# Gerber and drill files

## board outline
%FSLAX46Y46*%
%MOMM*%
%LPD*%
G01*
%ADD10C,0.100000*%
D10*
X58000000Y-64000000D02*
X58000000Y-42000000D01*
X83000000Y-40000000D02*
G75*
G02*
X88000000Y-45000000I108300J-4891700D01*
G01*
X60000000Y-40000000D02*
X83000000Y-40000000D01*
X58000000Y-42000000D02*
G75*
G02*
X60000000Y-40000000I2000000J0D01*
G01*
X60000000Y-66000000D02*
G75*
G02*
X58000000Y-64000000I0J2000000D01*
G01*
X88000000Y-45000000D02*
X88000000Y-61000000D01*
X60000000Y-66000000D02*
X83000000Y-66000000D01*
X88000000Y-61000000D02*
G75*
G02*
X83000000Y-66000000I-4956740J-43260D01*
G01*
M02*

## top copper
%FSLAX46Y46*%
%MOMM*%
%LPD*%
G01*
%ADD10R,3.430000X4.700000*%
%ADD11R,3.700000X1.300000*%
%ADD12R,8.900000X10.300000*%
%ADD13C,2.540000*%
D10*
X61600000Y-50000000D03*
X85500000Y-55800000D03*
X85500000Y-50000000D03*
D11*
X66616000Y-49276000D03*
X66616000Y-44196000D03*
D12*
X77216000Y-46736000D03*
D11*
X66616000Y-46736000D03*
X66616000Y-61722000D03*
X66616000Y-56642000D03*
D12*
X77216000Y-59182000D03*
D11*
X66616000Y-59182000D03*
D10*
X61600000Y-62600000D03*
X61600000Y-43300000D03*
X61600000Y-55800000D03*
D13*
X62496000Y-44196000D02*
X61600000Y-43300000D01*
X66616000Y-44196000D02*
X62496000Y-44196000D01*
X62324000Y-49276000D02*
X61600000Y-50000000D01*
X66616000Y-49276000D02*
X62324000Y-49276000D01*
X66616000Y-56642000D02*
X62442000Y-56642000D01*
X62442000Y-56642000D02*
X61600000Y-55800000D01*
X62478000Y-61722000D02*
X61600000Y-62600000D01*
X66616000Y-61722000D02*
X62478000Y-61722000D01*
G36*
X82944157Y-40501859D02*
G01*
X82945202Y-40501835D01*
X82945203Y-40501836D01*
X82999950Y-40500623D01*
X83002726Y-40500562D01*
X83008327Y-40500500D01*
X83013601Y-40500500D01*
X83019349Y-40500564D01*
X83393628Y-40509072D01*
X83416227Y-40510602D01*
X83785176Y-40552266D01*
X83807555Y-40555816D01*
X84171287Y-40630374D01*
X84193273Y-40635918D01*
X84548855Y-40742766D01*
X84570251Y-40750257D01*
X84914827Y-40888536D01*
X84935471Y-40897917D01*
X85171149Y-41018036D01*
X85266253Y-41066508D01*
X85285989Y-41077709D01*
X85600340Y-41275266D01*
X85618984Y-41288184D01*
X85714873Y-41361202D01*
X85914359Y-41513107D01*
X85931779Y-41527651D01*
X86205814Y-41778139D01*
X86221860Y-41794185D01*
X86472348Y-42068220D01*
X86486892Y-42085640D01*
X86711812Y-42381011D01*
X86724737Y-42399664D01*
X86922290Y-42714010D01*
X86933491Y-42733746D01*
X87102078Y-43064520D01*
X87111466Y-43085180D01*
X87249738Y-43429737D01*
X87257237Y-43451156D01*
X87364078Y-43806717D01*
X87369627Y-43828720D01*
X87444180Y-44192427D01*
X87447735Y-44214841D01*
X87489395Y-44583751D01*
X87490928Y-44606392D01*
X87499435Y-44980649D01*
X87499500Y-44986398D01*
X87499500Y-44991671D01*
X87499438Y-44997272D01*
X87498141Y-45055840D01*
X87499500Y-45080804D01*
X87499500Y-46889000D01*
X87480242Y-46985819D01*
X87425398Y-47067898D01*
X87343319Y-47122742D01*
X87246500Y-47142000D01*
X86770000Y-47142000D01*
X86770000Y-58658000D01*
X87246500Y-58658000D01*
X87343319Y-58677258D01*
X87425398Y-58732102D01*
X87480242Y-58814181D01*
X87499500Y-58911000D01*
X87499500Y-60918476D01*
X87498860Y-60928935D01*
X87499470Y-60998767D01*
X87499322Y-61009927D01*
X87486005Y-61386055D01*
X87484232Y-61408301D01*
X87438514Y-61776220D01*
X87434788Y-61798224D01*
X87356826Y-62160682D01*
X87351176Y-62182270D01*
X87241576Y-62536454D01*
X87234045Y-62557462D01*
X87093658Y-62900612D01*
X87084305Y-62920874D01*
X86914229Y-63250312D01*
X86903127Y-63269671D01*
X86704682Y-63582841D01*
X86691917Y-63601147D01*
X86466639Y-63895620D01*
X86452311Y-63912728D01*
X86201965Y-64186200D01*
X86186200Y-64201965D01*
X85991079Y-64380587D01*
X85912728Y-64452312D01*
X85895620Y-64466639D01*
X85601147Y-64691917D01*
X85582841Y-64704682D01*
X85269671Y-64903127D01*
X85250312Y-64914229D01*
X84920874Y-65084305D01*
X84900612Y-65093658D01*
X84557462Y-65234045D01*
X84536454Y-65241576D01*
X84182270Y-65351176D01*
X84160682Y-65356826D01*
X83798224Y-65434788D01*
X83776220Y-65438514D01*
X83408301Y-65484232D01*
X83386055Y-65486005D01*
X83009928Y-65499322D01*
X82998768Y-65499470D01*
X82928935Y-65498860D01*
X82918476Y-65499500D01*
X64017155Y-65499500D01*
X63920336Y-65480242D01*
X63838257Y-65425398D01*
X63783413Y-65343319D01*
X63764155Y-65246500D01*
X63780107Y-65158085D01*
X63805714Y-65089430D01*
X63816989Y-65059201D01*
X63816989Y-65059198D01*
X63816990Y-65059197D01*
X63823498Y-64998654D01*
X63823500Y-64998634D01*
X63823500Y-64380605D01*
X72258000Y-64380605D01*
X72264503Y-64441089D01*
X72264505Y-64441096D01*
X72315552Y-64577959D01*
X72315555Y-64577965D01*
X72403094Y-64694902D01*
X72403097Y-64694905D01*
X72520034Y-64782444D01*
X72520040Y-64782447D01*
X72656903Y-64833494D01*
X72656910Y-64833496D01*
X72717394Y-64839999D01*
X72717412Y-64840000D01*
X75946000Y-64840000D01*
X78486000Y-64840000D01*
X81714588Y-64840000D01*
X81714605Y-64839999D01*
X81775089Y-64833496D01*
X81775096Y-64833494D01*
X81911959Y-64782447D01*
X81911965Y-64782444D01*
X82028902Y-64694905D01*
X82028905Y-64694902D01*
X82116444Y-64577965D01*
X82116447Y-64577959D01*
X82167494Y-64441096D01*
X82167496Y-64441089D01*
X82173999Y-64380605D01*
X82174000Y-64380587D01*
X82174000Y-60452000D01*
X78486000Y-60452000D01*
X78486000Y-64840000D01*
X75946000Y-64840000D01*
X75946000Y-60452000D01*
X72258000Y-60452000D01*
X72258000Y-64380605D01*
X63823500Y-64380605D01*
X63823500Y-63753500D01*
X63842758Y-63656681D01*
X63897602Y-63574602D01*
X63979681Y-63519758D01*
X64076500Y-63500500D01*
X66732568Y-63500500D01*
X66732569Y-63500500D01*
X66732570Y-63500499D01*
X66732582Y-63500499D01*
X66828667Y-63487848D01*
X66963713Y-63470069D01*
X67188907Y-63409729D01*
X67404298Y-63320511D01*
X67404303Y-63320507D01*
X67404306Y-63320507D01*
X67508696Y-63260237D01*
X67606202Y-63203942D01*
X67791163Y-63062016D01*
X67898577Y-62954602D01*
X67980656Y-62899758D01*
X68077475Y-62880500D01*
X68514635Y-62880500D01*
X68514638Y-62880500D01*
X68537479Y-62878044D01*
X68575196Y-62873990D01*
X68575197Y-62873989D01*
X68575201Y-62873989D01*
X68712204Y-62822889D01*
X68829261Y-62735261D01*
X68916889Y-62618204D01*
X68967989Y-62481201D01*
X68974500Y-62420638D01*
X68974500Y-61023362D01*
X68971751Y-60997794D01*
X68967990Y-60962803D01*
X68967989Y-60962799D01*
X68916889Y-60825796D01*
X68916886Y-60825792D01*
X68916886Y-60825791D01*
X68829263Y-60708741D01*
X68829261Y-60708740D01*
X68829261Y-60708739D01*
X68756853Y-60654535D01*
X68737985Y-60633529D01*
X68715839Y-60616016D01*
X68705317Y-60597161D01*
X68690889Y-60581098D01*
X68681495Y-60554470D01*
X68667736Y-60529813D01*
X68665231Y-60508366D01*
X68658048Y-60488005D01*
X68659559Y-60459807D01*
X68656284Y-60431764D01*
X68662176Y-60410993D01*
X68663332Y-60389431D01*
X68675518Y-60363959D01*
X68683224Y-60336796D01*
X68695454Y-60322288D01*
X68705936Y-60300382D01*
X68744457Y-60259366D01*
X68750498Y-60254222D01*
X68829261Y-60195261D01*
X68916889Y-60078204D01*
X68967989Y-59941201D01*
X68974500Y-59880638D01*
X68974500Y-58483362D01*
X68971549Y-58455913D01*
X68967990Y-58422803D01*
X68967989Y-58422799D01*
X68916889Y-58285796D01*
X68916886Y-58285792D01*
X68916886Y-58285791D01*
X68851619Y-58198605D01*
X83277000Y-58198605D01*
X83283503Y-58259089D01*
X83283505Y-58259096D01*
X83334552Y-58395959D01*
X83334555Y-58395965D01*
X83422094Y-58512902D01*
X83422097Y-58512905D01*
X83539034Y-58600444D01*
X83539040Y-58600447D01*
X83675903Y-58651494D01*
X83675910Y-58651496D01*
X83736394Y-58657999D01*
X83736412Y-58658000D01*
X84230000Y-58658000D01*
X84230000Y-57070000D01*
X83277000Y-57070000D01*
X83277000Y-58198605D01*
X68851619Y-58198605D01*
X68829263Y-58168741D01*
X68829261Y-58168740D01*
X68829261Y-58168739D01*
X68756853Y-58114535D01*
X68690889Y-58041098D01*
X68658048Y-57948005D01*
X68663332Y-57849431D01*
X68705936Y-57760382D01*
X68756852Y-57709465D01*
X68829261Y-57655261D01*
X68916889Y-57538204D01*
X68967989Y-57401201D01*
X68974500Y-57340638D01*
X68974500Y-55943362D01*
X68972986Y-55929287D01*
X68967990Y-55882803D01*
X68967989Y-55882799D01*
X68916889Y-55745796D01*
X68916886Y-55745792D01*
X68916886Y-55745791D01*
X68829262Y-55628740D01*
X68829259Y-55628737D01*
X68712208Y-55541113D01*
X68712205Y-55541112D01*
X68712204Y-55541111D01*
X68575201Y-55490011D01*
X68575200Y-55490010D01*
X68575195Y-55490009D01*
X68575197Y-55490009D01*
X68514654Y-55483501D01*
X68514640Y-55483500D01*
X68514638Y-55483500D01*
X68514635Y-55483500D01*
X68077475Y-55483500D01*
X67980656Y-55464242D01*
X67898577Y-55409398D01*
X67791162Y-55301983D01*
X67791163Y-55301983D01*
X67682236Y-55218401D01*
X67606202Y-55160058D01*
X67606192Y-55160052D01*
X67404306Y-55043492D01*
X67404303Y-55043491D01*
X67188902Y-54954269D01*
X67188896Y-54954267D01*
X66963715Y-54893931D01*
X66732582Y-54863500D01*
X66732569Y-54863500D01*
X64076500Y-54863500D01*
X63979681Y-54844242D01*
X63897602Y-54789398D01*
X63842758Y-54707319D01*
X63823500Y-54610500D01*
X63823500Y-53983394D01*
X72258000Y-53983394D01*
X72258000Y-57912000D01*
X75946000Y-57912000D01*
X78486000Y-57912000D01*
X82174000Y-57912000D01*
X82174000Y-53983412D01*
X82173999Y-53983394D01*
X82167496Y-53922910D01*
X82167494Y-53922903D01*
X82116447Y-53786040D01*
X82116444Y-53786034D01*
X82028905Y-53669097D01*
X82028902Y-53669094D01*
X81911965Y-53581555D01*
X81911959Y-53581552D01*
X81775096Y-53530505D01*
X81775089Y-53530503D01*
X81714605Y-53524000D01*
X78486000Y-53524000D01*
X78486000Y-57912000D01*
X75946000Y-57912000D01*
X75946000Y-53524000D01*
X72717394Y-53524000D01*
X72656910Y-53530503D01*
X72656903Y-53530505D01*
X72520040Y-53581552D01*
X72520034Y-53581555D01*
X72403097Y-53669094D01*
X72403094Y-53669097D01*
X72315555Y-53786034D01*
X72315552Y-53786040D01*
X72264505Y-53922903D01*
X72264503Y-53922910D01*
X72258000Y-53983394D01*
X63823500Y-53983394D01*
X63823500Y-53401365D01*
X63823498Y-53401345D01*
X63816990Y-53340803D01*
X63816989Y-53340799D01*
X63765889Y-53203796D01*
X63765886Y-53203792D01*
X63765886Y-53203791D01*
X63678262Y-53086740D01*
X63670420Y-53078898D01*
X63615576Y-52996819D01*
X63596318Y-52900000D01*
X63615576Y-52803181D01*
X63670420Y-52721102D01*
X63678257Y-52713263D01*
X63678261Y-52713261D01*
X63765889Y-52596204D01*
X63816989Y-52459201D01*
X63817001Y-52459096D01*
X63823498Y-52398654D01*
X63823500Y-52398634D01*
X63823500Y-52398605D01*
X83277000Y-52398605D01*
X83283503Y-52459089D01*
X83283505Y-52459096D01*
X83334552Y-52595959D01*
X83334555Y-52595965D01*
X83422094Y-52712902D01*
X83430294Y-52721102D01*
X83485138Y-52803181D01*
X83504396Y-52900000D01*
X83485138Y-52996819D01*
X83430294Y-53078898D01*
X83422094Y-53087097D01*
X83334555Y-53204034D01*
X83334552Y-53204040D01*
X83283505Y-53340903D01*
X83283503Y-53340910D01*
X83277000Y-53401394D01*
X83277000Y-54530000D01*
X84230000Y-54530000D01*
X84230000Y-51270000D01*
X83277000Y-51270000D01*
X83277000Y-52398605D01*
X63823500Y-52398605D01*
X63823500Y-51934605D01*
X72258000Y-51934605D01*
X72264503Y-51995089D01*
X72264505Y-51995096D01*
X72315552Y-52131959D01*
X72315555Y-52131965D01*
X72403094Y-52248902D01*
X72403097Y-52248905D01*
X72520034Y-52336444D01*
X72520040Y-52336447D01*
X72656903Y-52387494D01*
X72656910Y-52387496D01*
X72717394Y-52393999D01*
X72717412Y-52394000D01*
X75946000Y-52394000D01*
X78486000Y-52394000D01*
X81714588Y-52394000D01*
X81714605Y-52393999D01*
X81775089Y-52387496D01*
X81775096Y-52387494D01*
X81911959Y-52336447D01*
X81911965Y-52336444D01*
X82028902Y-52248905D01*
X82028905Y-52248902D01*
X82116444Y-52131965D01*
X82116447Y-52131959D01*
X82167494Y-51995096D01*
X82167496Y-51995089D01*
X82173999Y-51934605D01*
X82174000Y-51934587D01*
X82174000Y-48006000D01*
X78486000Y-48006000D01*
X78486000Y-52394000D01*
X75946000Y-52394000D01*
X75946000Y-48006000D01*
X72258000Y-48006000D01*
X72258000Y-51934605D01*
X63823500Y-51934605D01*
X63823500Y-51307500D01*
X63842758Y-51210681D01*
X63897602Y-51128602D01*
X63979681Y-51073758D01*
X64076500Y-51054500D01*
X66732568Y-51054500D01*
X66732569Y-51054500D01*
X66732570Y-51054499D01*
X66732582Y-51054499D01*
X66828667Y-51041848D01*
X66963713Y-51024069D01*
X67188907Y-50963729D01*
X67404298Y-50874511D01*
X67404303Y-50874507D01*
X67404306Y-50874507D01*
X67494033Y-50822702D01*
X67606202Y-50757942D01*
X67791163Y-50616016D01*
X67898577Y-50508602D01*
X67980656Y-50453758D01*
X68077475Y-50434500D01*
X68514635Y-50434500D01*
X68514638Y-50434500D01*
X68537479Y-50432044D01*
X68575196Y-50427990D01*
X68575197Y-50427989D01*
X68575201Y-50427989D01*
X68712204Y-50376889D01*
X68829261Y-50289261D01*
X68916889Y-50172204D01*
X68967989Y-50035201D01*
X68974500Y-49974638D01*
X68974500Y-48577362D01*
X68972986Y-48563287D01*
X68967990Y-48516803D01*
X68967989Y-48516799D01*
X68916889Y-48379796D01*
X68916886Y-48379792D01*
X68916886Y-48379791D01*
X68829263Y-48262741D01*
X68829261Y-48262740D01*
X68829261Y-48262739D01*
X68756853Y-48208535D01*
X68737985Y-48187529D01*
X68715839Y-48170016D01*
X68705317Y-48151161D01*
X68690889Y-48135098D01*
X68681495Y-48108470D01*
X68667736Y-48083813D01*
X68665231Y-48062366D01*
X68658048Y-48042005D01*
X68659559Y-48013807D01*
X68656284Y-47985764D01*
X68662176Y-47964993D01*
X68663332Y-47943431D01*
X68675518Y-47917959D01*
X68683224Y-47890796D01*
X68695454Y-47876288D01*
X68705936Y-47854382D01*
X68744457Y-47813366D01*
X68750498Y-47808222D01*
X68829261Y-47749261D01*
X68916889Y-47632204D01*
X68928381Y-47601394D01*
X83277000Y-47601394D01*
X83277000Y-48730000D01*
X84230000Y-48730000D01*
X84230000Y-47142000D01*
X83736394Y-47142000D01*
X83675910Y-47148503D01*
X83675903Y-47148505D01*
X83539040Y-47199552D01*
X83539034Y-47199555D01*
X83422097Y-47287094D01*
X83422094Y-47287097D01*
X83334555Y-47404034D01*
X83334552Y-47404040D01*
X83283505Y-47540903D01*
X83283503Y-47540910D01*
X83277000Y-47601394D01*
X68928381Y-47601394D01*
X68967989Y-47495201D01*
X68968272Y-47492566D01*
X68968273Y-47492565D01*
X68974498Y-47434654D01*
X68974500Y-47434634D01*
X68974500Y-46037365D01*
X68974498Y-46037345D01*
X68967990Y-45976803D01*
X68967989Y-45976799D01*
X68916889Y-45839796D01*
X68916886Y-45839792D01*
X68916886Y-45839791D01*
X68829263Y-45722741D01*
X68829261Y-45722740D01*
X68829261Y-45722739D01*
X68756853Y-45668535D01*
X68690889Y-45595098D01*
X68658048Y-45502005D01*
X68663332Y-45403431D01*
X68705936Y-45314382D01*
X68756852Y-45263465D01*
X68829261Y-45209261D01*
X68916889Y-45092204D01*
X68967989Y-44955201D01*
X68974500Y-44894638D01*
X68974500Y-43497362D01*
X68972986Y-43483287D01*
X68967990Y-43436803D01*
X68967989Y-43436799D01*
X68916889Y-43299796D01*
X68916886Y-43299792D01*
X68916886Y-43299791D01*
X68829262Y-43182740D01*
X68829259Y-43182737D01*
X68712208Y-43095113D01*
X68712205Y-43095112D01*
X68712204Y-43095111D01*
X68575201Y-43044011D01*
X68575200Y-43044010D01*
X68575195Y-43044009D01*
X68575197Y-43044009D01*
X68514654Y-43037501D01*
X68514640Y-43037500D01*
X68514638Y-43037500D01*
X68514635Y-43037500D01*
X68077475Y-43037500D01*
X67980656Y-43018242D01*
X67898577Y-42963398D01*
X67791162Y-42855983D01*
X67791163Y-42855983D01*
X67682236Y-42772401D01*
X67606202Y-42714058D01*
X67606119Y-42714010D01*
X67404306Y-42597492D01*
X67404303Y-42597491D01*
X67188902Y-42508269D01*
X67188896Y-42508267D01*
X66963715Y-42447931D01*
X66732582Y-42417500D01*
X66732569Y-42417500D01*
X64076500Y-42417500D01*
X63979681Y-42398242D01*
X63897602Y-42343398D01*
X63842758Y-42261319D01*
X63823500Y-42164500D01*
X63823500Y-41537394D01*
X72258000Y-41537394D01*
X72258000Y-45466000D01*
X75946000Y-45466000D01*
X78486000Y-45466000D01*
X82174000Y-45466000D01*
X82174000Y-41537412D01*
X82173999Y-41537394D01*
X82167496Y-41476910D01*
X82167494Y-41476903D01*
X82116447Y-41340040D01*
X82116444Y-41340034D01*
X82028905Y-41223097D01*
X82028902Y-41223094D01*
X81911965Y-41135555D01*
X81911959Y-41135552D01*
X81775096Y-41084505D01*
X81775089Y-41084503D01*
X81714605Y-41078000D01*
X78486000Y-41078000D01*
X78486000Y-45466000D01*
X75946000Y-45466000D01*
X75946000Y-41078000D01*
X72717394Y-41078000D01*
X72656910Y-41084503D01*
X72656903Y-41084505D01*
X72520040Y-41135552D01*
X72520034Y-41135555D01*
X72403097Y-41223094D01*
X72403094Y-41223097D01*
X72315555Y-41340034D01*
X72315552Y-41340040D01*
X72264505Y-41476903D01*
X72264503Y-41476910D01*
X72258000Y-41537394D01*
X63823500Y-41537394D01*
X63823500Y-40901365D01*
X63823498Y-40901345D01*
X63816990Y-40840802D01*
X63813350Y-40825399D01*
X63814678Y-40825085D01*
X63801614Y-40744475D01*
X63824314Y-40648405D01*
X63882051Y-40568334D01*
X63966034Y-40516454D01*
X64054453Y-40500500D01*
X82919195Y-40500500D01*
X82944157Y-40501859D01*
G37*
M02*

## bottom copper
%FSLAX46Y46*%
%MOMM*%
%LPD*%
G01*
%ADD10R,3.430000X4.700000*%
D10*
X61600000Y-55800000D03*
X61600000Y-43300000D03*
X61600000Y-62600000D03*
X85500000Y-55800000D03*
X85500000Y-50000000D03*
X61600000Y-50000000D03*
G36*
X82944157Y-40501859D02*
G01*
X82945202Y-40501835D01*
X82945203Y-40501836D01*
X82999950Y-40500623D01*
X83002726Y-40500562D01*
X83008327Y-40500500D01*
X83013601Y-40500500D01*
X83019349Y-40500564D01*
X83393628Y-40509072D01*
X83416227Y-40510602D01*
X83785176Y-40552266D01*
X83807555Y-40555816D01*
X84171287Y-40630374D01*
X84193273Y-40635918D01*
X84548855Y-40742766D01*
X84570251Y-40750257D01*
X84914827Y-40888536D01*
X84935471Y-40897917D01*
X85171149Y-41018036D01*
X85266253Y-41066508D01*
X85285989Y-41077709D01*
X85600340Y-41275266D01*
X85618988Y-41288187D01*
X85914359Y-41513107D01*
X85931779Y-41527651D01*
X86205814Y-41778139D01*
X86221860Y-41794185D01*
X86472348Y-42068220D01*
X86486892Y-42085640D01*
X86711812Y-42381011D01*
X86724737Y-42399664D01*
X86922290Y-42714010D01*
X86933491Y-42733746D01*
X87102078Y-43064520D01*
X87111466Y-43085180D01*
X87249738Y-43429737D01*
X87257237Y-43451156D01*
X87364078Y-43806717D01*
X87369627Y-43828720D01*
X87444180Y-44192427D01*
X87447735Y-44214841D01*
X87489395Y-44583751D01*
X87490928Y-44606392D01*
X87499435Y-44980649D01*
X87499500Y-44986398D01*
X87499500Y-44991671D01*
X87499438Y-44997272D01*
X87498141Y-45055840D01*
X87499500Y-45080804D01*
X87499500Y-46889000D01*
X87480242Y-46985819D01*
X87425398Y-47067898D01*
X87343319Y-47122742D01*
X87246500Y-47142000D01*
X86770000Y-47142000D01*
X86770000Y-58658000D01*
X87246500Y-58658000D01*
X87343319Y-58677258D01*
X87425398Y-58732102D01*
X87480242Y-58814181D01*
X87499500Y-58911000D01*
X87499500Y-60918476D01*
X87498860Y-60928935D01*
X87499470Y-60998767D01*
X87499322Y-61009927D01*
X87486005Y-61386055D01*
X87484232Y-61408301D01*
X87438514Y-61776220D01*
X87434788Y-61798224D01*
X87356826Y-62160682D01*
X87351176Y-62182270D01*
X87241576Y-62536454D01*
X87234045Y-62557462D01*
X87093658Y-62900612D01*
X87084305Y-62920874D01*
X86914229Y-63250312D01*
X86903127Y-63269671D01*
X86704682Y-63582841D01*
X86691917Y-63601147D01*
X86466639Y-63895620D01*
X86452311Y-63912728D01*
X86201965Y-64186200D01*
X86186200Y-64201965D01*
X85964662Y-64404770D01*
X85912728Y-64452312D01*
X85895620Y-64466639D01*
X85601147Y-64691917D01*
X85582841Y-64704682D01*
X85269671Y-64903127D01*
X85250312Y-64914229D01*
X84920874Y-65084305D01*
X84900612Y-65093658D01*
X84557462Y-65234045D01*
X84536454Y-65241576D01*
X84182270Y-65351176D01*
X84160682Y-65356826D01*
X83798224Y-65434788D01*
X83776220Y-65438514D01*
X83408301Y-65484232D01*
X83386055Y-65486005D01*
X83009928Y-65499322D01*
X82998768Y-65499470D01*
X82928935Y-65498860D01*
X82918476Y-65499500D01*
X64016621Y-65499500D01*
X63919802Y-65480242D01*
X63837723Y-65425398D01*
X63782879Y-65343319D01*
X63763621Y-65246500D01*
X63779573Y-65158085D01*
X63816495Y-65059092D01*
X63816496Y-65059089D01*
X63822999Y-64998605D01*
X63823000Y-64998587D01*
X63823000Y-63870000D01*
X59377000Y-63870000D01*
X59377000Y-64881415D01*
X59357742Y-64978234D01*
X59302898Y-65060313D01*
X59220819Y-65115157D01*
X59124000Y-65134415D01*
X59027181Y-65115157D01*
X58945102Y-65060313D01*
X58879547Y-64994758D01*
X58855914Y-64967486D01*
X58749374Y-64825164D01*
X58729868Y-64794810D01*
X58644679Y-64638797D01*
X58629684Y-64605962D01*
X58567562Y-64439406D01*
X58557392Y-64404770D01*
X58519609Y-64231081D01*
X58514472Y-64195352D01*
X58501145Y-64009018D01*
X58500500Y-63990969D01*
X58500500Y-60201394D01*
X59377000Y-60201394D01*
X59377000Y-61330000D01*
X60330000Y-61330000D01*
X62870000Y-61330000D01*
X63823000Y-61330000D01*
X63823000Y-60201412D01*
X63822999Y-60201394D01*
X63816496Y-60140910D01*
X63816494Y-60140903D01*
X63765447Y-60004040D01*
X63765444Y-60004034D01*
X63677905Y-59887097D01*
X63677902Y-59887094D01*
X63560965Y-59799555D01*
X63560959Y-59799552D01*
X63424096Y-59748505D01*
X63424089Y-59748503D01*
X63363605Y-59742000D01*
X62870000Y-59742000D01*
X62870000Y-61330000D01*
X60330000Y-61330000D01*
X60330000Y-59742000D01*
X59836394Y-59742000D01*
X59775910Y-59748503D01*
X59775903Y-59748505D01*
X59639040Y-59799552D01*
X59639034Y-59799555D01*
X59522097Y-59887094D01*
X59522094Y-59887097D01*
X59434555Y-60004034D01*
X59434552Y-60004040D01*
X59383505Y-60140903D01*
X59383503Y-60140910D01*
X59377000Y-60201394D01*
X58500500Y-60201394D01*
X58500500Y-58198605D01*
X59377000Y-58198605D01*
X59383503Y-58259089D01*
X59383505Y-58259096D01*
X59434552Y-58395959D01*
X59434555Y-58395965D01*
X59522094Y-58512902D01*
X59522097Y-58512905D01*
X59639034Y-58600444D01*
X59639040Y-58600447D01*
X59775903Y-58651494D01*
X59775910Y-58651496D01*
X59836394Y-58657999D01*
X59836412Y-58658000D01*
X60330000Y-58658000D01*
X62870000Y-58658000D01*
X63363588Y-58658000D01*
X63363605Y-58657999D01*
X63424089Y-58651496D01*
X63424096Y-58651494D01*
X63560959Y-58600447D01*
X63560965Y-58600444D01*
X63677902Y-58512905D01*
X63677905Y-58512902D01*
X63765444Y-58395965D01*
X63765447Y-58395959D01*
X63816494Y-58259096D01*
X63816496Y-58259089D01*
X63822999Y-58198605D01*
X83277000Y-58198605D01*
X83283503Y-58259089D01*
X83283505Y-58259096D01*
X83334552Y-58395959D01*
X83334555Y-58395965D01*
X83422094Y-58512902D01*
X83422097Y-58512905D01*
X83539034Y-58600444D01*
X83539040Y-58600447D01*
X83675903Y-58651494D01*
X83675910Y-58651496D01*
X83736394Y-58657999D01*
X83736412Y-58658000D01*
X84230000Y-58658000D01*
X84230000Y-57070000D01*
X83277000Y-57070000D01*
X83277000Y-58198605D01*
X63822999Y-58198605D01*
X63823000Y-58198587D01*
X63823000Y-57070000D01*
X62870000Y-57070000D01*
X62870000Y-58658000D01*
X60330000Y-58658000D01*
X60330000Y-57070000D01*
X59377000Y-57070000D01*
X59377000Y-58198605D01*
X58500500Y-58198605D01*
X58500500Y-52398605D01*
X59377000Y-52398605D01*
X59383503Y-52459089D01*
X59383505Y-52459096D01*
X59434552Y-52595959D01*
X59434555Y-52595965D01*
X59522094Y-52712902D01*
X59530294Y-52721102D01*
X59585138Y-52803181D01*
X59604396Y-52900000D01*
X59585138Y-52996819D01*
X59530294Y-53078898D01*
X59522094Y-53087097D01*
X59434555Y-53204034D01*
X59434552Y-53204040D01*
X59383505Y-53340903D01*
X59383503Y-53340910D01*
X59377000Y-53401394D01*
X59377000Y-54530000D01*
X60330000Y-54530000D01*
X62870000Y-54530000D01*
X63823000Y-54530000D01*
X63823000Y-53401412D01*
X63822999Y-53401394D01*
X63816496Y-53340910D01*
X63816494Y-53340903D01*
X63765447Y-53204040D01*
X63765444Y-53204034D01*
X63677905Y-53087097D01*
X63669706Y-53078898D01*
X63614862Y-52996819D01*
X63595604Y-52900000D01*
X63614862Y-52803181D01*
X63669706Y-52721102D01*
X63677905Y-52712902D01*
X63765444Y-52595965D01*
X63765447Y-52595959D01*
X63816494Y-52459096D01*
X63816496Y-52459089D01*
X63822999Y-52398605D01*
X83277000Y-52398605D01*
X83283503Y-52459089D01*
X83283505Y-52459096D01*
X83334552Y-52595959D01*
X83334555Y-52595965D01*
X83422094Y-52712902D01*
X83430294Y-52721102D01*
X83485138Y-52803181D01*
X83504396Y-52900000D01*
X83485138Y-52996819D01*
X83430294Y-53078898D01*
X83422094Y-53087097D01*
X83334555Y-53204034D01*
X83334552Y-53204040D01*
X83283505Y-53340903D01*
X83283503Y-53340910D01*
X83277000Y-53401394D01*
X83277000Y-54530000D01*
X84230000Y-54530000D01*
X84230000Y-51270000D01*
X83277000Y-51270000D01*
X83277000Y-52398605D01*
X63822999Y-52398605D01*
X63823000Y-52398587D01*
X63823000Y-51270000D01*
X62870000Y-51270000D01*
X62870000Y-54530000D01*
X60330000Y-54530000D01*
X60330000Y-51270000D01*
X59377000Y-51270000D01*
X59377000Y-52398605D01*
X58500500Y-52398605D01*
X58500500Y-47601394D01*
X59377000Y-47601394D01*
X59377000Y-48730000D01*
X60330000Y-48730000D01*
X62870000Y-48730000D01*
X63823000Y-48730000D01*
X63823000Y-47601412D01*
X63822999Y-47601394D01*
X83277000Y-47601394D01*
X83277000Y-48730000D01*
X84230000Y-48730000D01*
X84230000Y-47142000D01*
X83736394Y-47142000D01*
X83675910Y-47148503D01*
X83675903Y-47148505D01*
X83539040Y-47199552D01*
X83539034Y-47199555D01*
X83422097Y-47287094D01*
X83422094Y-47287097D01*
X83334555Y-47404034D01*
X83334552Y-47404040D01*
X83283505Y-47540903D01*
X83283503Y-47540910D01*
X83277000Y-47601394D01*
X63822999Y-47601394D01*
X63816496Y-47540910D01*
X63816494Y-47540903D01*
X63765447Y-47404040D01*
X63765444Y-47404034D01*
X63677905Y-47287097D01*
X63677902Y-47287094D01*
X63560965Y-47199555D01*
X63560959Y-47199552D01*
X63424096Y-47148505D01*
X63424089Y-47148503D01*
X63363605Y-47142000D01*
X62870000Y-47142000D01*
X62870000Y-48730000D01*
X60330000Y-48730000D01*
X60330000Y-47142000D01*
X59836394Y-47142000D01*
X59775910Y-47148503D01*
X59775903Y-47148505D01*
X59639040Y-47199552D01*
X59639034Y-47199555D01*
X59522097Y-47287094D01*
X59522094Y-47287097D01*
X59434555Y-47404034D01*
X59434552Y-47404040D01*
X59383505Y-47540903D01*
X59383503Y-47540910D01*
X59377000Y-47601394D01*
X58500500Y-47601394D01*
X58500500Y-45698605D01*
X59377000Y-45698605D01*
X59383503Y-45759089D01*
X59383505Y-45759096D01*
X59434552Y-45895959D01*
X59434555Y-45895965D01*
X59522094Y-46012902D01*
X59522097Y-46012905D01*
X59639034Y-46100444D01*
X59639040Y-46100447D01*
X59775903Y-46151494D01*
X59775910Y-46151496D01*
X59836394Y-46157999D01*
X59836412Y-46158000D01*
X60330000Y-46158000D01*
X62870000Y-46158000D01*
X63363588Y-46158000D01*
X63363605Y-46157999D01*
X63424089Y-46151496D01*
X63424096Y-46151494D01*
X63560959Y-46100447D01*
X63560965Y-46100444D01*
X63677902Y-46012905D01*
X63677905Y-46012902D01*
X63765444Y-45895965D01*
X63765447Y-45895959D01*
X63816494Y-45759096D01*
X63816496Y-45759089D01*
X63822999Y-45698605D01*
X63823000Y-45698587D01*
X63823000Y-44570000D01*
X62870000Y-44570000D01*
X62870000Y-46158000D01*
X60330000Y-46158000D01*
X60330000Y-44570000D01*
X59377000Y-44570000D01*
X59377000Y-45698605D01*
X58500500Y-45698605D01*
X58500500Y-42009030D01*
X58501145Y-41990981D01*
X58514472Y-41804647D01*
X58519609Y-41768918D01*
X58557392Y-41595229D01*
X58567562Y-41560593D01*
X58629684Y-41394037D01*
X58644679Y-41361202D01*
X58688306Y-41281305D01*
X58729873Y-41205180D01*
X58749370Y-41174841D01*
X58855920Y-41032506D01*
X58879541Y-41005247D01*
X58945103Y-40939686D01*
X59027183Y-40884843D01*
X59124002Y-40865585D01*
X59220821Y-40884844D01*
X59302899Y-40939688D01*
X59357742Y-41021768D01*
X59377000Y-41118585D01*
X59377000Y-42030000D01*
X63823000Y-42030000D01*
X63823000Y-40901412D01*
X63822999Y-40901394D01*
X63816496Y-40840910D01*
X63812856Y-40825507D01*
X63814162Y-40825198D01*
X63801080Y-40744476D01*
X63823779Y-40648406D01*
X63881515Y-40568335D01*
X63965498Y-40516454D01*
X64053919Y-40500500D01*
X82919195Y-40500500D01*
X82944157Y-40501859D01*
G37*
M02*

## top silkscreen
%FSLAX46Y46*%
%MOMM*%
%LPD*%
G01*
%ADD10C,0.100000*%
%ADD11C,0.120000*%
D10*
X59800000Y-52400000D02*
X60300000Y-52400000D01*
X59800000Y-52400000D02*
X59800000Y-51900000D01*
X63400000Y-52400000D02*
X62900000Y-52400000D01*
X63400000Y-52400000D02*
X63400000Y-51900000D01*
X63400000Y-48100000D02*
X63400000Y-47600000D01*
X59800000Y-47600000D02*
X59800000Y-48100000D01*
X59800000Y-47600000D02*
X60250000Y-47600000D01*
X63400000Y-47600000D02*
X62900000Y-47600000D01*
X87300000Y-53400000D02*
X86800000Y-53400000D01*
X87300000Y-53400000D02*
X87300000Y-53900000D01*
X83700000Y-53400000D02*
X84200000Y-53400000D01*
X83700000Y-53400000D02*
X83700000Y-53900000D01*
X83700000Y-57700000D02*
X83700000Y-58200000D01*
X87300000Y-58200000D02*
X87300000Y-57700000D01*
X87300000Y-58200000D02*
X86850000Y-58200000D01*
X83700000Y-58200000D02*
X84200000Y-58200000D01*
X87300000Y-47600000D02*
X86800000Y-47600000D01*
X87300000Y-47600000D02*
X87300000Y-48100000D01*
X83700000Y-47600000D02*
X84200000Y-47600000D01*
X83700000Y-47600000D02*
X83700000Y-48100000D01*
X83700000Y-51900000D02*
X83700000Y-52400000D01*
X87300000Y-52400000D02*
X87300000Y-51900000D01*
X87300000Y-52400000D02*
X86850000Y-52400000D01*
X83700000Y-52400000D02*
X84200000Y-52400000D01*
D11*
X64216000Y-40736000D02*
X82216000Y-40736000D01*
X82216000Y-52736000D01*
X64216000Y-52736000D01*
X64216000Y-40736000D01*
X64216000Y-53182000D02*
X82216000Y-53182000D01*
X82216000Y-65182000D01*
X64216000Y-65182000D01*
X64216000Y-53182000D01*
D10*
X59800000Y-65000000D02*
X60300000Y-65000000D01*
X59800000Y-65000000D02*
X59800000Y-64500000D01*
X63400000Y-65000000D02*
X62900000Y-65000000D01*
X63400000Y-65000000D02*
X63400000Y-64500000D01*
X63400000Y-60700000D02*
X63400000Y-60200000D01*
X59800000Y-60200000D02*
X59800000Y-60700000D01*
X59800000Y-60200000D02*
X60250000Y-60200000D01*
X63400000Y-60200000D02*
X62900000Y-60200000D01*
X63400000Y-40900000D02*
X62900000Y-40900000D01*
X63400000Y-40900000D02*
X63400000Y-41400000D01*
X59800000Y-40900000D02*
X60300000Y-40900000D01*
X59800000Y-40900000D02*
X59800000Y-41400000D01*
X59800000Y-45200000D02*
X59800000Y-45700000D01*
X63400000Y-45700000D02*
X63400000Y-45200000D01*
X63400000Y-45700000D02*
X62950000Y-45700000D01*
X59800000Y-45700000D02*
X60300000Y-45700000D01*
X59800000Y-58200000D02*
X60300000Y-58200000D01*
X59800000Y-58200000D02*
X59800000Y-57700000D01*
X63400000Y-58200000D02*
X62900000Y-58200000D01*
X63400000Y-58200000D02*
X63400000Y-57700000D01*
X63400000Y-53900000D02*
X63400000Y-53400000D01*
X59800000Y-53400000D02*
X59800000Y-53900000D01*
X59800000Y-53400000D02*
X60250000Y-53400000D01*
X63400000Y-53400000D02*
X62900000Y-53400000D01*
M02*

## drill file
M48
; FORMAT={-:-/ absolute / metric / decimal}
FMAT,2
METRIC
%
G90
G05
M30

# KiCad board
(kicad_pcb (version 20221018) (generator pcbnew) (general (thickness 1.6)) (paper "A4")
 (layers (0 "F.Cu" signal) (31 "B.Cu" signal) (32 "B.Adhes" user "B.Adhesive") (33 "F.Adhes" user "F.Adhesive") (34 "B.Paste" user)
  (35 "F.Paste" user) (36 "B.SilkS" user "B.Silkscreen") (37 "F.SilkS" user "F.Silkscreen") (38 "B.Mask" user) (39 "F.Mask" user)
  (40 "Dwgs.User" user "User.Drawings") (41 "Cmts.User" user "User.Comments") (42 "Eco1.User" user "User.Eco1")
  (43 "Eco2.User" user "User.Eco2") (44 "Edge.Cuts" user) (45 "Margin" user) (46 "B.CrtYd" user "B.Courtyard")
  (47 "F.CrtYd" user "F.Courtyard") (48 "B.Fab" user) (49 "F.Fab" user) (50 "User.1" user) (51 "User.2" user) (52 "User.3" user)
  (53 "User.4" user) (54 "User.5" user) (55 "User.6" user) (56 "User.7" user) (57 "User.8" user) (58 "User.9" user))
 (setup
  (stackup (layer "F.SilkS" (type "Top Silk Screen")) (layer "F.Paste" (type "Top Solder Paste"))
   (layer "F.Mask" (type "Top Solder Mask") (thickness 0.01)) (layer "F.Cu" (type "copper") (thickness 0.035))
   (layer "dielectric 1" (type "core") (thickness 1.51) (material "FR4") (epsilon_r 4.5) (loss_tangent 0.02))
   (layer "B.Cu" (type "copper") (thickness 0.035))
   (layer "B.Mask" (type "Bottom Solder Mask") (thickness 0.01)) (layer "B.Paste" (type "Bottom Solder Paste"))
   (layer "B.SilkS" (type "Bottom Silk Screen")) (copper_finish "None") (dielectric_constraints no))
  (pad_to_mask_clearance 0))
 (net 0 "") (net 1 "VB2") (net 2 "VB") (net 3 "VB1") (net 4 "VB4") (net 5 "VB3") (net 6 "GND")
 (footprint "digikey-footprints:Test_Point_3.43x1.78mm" (layer "F.Cu") (at 61.6 50 90)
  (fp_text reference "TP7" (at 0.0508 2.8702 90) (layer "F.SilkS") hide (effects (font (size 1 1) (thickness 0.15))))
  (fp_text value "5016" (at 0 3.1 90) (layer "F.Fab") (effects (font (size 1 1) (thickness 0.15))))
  (fp_line (start -2.4 -1.8) (end -2.4 -1.3) (stroke (width 0.1) (type solid)) (layer "F.SilkS"))
  (fp_line (start -2.4 -1.8) (end -1.9 -1.8) (stroke (width 0.1) (type solid)) (layer "F.SilkS"))
  (fp_line (start -2.4 1.8) (end -2.4 1.3) (stroke (width 0.1) (type solid)) (layer "F.SilkS"))
  (fp_line (start -2.4 1.8) (end -1.9 1.8) (stroke (width 0.1) (type solid)) (layer "F.SilkS"))
  (fp_line (start 1.9 1.8) (end 2.4 1.8) (stroke (width 0.1) (type solid)) (layer "F.SilkS"))
  (fp_line (start 2.4 -1.8) (end 1.9 -1.8) (stroke (width 0.1) (type solid)) (layer "F.SilkS"))
  (fp_line (start 2.4 -1.8) (end 2.4 -1.35) (stroke (width 0.1) (type solid)) (layer "F.SilkS"))
  (fp_line (start 2.4 1.8) (end 2.4 1.3) (stroke (width 0.1) (type solid)) (layer "F.SilkS"))
  (pad "1" smd rect (at 0 0 90) (size 4.7 3.43) (layers "F.Cu" "F.Paste" "F.Mask") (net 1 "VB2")))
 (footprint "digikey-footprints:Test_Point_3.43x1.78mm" (layer "F.Cu") (at 85.5 55.8 -90)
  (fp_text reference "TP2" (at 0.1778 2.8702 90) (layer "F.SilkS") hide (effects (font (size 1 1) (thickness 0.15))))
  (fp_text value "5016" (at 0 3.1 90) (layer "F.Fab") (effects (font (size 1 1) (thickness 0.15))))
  (fp_line (start -2.4 -1.8) (end -2.4 -1.3) (stroke (width 0.1) (type solid)) (layer "F.SilkS"))
  (fp_line (start -2.4 -1.8) (end -1.9 -1.8) (stroke (width 0.1) (type solid)) (layer "F.SilkS"))
  (fp_line (start -2.4 1.8) (end -2.4 1.3) (stroke (width 0.1) (type solid)) (layer "F.SilkS"))
  (fp_line (start -2.4 1.8) (end -1.9 1.8) (stroke (width 0.1) (type solid)) (layer "F.SilkS"))
  (fp_line (start 1.9 1.8) (end 2.4 1.8) (stroke (width 0.1) (type solid)) (layer "F.SilkS"))
  (fp_line (start 2.4 -1.8) (end 1.9 -1.8) (stroke (width 0.1) (type solid)) (layer "F.SilkS"))
  (fp_line (start 2.4 -1.8) (end 2.4 -1.35) (stroke (width 0.1) (type solid)) (layer "F.SilkS"))
  (fp_line (start 2.4 1.8) (end 2.4 1.3) (stroke (width 0.1) (type solid)) (layer "F.SilkS"))
  (pad "1" smd rect (at 0 0 270) (size 4.7 3.43) (layers "F.Cu" "F.Paste" "F.Mask") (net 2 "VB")))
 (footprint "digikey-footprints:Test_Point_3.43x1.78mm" (layer "F.Cu") (at 85.5 50 -90)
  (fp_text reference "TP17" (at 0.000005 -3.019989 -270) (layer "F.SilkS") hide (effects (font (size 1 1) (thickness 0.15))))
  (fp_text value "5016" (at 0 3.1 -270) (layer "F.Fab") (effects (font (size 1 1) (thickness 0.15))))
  (fp_line (start -2.4 -1.8) (end -2.4 -1.3) (stroke (width 0.1) (type solid)) (layer "F.SilkS"))
  (fp_line (start -2.4 -1.8) (end -1.9 -1.8) (stroke (width 0.1) (type solid)) (layer "F.SilkS"))
  (fp_line (start -2.4 1.8) (end -2.4 1.3) (stroke (width 0.1) (type solid)) (layer "F.SilkS"))
  (fp_line (start -2.4 1.8) (end -1.9 1.8) (stroke (width 0.1) (type solid)) (layer "F.SilkS"))
  (fp_line (start 1.9 1.8) (end 2.4 1.8) (stroke (width 0.1) (type solid)) (layer "F.SilkS"))
  (fp_line (start 2.4 -1.8) (end 1.9 -1.8) (stroke (width 0.1) (type solid)) (layer "F.SilkS"))
  (fp_line (start 2.4 -1.8) (end 2.4 -1.35) (stroke (width 0.1) (type solid)) (layer "F.SilkS"))
  (fp_line (start 2.4 1.8) (end 2.4 1.3) (stroke (width 0.1) (type solid)) (layer "F.SilkS"))
  (pad "1" smd rect (at 0 0 270) (size 4.7 3.43) (layers "F.Cu" "F.Paste" "F.Mask") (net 2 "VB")))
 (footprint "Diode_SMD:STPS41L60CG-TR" (layer "F.Cu") (at 77.216 46.736 180)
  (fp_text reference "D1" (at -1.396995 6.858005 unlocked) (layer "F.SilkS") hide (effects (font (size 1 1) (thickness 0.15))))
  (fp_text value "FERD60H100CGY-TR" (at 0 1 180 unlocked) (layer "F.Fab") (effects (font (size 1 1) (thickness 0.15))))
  (fp_rect (start -5 -6) (end 13 6) (stroke (width 0.12) (type solid)) (fill none) (layer "F.SilkS"))
  (pad "1" smd rect (at 10.6 -2.54 180) (size 3.7 1.3) (layers "F.Cu" "F.Paste" "F.Mask") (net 1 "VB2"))
  (pad "2" smd rect (at 10.6 2.54 180) (size 3.7 1.3) (layers "F.Cu" "F.Paste" "F.Mask") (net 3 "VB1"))
  (pad "3" smd rect (at 0 0 180) (size 8.9 10.3) (layers "F.Cu" "F.Paste" "F.Mask") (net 2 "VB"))
  (pad "4" smd rect (at 10.6 0 180) (size 3.7 1.3) (layers "F.Cu" "F.Paste" "F.Mask")))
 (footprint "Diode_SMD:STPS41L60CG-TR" (layer "F.Cu") (at 77.216 59.182 180)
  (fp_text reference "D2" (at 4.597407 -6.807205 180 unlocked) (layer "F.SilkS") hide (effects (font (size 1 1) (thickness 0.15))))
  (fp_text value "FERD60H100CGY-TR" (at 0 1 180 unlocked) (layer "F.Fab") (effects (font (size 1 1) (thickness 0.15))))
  (fp_rect (start -5 -6) (end 13 6) (stroke (width 0.12) (type solid)) (fill none) (layer "F.SilkS"))
  (pad "1" smd rect (at 10.6 -2.54 180) (size 3.7 1.3) (layers "F.Cu" "F.Paste" "F.Mask") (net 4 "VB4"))
  (pad "2" smd rect (at 10.6 2.54 180) (size 3.7 1.3) (layers "F.Cu" "F.Paste" "F.Mask") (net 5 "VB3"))
  (pad "3" smd rect (at 0 0 180) (size 8.9 10.3) (layers "F.Cu" "F.Paste" "F.Mask") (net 2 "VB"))
  (pad "4" smd rect (at 10.6 0 180) (size 3.7 1.3) (layers "F.Cu" "F.Paste" "F.Mask")))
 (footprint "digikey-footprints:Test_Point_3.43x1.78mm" (layer "F.Cu") (at 61.6 62.6 90)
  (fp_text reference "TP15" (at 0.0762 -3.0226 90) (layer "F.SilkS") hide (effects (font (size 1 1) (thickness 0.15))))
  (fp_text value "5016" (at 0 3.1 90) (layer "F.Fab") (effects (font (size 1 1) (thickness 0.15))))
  (fp_line (start -2.4 -1.8) (end -2.4 -1.3) (stroke (width 0.1) (type solid)) (layer "F.SilkS"))
  (fp_line (start -2.4 -1.8) (end -1.9 -1.8) (stroke (width 0.1) (type solid)) (layer "F.SilkS"))
  (fp_line (start -2.4 1.8) (end -2.4 1.3) (stroke (width 0.1) (type solid)) (layer "F.SilkS"))
  (fp_line (start -2.4 1.8) (end -1.9 1.8) (stroke (width 0.1) (type solid)) (layer "F.SilkS"))
  (fp_line (start 1.9 1.8) (end 2.4 1.8) (stroke (width 0.1) (type solid)) (layer "F.SilkS"))
  (fp_line (start 2.4 -1.8) (end 1.9 -1.8) (stroke (width 0.1) (type solid)) (layer "F.SilkS"))
  (fp_line (start 2.4 -1.8) (end 2.4 -1.35) (stroke (width 0.1) (type solid)) (layer "F.SilkS"))
  (fp_line (start 2.4 1.8) (end 2.4 1.3) (stroke (width 0.1) (type solid)) (layer "F.SilkS"))
  (pad "1" smd rect (at 0 0 90) (size 4.7 3.43) (layers "F.Cu" "F.Paste" "F.Mask") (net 4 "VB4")))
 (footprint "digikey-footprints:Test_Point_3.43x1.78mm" (layer "F.Cu") (at 61.6 43.3 -90)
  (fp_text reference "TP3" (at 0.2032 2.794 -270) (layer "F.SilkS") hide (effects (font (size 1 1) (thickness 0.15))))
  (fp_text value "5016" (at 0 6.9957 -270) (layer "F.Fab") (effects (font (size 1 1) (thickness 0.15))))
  (fp_line (start -2.4 -1.8) (end -2.4 -1.3) (stroke (width 0.1) (type solid)) (layer "F.SilkS"))
  (fp_line (start -2.4 -1.8) (end -1.9 -1.8) (stroke (width 0.1) (type solid)) (layer "F.SilkS"))
  (fp_line (start -2.4 1.8) (end -2.4 1.3) (stroke (width 0.1) (type solid)) (layer "F.SilkS"))
  (fp_line (start -2.4 1.8) (end -1.9 1.8) (stroke (width 0.1) (type solid)) (layer "F.SilkS"))
  (fp_line (start 1.9 1.8) (end 2.4 1.8) (stroke (width 0.1) (type solid)) (layer "F.SilkS"))
  (fp_line (start 2.4 -1.8) (end 1.9 -1.8) (stroke (width 0.1) (type solid)) (layer "F.SilkS"))
  (fp_line (start 2.4 -1.8) (end 2.4 -1.35) (stroke (width 0.1) (type solid)) (layer "F.SilkS"))
  (fp_line (start 2.4 1.8) (end 2.4 1.3) (stroke (width 0.1) (type solid)) (layer "F.SilkS"))
  (pad "1" smd rect (at 0 0 270) (size 4.7 3.43) (layers "F.Cu" "F.Paste" "F.Mask") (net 3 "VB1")))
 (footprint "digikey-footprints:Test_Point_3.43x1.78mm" (layer "F.Cu") (at 61.6 55.8 90)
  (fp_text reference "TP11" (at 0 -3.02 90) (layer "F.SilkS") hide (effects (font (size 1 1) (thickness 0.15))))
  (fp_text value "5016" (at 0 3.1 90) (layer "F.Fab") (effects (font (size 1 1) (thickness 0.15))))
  (fp_line (start -2.4 -1.8) (end -2.4 -1.3) (stroke (width 0.1) (type solid)) (layer "F.SilkS"))
  (fp_line (start -2.4 -1.8) (end -1.9 -1.8) (stroke (width 0.1) (type solid)) (layer "F.SilkS"))
  (fp_line (start -2.4 1.8) (end -2.4 1.3) (stroke (width 0.1) (type solid)) (layer "F.SilkS"))
  (fp_line (start -2.4 1.8) (end -1.9 1.8) (stroke (width 0.1) (type solid)) (layer "F.SilkS"))
  (fp_line (start 1.9 1.8) (end 2.4 1.8) (stroke (width 0.1) (type solid)) (layer "F.SilkS"))
  (fp_line (start 2.4 -1.8) (end 1.9 -1.8) (stroke (width 0.1) (type solid)) (layer "F.SilkS"))
  (fp_line (start 2.4 -1.8) (end 2.4 -1.35) (stroke (width 0.1) (type solid)) (layer "F.SilkS"))
  (fp_line (start 2.4 1.8) (end 2.4 1.3) (stroke (width 0.1) (type solid)) (layer "F.SilkS"))
  (pad "1" smd rect (at 0 0 90) (size 4.7 3.43) (layers "F.Cu" "F.Paste" "F.Mask") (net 5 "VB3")))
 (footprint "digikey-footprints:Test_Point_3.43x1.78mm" (layer "B.Cu") (at 61.6 55.8 -90)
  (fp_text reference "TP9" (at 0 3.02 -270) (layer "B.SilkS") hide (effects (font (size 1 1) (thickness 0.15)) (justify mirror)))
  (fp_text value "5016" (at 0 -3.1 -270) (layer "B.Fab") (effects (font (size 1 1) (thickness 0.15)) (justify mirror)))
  (pad "1" smd rect (at 0 0 270) (size 4.7 3.43) (layers "B.Cu" "B.Paste" "B.Mask") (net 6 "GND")))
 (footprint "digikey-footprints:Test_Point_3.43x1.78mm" (layer "B.Cu") (at 61.6 43.3 -90)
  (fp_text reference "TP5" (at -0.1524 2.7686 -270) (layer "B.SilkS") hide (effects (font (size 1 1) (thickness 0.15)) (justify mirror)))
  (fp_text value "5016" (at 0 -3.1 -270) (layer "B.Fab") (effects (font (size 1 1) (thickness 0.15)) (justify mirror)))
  (pad "1" smd rect (at 0 0 270) (size 4.7 3.43) (layers "B.Cu" "B.Paste" "B.Mask") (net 6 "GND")))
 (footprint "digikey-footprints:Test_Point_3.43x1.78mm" (layer "B.Cu") (at 61.6 62.6 90)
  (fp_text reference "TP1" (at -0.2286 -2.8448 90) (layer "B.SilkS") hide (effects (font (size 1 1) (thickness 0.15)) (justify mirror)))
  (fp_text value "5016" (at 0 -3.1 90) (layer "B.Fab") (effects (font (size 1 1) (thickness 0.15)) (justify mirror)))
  (pad "1" smd rect (at 0 0 90) (size 4.7 3.43) (layers "B.Cu" "B.Paste" "B.Mask") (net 6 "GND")))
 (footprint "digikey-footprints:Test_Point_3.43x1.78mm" (layer "B.Cu") (at 85.5 55.8 -90)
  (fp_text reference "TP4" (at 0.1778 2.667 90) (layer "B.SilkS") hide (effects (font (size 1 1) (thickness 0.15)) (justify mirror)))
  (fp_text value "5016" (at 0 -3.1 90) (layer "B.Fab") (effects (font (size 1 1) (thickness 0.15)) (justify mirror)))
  (pad "1" smd rect (at 0 0 270) (size 4.7 3.43) (layers "B.Cu" "B.Paste" "B.Mask") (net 6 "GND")))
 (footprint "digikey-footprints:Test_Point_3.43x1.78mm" (layer "B.Cu") (at 85.5 50 -90)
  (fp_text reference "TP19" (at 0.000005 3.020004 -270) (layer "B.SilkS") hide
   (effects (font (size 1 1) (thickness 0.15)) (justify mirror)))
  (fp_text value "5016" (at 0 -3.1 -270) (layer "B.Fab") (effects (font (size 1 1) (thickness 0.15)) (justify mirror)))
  (pad "1" smd rect (at 0 0 270) (size 4.7 3.43) (layers "B.Cu" "B.Paste" "B.Mask") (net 6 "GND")))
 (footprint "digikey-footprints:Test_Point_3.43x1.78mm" (layer "B.Cu") (at 61.6 50 -90)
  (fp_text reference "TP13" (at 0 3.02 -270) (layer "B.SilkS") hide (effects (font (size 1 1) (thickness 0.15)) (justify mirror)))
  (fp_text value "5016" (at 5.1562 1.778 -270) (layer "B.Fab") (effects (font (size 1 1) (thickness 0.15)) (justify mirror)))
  (pad "1" smd rect (at 0 0 270) (size 4.7 3.43) (layers "B.Cu" "B.Paste" "B.Mask") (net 6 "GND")))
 (gr_line (start 58 64) (end 58 42) (stroke (width 0.1) (type solid)) (layer "Edge.Cuts"))
 (gr_arc (start 83 40) (mid 86.568105 41.431895) (end 88 45) (stroke (width 0.1) (type solid)) (layer "Edge.Cuts"))
 (gr_line (start 60 40) (end 83 40) (stroke (width 0.1) (type solid)) (layer "Edge.Cuts"))
 (gr_arc (start 58 42) (mid 58.585786 40.585786) (end 60 40) (stroke (width 0.1) (type solid)) (layer "Edge.Cuts"))
 (gr_arc (start 60 66) (mid 58.585786 65.414214) (end 58 64) (stroke (width 0.1) (type solid)) (layer "Edge.Cuts"))
 (gr_line (start 88 45) (end 88 61) (stroke (width 0.1) (type solid)) (layer "Edge.Cuts"))
 (gr_line (start 60 66) (end 83 66) (stroke (width 0.1) (type solid)) (layer "Edge.Cuts"))
 (gr_arc (start 88 61) (mid 86.548338 64.548337) (end 83 66) (stroke (width 0.1) (type solid)) (layer "Edge.Cuts"))
 (segment (start 62.496 44.196) (end 61.6 43.3) (width 2.54) (layer "F.Cu") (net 3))
 (segment (start 66.616 44.196) (end 62.496 44.196) (width 2.54) (layer "F.Cu") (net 3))
 (segment (start 62.324 49.276) (end 61.6 50) (width 2.54) (layer "F.Cu") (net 1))
 (segment (start 66.616 49.276) (end 62.324 49.276) (width 2.54) (layer "F.Cu") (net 1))
 (segment (start 66.616 56.642) (end 62.442 56.642) (width 2.54) (layer "F.Cu") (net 5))
 (segment (start 62.442 56.642) (end 61.6 55.8) (width 2.54) (layer "F.Cu") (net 5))
 (segment (start 62.478 61.722) (end 61.6 62.6) (width 2.54) (layer "F.Cu") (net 4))
 (segment (start 66.616 61.722) (end 62.478 61.722) (width 2.54) (layer "F.Cu") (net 4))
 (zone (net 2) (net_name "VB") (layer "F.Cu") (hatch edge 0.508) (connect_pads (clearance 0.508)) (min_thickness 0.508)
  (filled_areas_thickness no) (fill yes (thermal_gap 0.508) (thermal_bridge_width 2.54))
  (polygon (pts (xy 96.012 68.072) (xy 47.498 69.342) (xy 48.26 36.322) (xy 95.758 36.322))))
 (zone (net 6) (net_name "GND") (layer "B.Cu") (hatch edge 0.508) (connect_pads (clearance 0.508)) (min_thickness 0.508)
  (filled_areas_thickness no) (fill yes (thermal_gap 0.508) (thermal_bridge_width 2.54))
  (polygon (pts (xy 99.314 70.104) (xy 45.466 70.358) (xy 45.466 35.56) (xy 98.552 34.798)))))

